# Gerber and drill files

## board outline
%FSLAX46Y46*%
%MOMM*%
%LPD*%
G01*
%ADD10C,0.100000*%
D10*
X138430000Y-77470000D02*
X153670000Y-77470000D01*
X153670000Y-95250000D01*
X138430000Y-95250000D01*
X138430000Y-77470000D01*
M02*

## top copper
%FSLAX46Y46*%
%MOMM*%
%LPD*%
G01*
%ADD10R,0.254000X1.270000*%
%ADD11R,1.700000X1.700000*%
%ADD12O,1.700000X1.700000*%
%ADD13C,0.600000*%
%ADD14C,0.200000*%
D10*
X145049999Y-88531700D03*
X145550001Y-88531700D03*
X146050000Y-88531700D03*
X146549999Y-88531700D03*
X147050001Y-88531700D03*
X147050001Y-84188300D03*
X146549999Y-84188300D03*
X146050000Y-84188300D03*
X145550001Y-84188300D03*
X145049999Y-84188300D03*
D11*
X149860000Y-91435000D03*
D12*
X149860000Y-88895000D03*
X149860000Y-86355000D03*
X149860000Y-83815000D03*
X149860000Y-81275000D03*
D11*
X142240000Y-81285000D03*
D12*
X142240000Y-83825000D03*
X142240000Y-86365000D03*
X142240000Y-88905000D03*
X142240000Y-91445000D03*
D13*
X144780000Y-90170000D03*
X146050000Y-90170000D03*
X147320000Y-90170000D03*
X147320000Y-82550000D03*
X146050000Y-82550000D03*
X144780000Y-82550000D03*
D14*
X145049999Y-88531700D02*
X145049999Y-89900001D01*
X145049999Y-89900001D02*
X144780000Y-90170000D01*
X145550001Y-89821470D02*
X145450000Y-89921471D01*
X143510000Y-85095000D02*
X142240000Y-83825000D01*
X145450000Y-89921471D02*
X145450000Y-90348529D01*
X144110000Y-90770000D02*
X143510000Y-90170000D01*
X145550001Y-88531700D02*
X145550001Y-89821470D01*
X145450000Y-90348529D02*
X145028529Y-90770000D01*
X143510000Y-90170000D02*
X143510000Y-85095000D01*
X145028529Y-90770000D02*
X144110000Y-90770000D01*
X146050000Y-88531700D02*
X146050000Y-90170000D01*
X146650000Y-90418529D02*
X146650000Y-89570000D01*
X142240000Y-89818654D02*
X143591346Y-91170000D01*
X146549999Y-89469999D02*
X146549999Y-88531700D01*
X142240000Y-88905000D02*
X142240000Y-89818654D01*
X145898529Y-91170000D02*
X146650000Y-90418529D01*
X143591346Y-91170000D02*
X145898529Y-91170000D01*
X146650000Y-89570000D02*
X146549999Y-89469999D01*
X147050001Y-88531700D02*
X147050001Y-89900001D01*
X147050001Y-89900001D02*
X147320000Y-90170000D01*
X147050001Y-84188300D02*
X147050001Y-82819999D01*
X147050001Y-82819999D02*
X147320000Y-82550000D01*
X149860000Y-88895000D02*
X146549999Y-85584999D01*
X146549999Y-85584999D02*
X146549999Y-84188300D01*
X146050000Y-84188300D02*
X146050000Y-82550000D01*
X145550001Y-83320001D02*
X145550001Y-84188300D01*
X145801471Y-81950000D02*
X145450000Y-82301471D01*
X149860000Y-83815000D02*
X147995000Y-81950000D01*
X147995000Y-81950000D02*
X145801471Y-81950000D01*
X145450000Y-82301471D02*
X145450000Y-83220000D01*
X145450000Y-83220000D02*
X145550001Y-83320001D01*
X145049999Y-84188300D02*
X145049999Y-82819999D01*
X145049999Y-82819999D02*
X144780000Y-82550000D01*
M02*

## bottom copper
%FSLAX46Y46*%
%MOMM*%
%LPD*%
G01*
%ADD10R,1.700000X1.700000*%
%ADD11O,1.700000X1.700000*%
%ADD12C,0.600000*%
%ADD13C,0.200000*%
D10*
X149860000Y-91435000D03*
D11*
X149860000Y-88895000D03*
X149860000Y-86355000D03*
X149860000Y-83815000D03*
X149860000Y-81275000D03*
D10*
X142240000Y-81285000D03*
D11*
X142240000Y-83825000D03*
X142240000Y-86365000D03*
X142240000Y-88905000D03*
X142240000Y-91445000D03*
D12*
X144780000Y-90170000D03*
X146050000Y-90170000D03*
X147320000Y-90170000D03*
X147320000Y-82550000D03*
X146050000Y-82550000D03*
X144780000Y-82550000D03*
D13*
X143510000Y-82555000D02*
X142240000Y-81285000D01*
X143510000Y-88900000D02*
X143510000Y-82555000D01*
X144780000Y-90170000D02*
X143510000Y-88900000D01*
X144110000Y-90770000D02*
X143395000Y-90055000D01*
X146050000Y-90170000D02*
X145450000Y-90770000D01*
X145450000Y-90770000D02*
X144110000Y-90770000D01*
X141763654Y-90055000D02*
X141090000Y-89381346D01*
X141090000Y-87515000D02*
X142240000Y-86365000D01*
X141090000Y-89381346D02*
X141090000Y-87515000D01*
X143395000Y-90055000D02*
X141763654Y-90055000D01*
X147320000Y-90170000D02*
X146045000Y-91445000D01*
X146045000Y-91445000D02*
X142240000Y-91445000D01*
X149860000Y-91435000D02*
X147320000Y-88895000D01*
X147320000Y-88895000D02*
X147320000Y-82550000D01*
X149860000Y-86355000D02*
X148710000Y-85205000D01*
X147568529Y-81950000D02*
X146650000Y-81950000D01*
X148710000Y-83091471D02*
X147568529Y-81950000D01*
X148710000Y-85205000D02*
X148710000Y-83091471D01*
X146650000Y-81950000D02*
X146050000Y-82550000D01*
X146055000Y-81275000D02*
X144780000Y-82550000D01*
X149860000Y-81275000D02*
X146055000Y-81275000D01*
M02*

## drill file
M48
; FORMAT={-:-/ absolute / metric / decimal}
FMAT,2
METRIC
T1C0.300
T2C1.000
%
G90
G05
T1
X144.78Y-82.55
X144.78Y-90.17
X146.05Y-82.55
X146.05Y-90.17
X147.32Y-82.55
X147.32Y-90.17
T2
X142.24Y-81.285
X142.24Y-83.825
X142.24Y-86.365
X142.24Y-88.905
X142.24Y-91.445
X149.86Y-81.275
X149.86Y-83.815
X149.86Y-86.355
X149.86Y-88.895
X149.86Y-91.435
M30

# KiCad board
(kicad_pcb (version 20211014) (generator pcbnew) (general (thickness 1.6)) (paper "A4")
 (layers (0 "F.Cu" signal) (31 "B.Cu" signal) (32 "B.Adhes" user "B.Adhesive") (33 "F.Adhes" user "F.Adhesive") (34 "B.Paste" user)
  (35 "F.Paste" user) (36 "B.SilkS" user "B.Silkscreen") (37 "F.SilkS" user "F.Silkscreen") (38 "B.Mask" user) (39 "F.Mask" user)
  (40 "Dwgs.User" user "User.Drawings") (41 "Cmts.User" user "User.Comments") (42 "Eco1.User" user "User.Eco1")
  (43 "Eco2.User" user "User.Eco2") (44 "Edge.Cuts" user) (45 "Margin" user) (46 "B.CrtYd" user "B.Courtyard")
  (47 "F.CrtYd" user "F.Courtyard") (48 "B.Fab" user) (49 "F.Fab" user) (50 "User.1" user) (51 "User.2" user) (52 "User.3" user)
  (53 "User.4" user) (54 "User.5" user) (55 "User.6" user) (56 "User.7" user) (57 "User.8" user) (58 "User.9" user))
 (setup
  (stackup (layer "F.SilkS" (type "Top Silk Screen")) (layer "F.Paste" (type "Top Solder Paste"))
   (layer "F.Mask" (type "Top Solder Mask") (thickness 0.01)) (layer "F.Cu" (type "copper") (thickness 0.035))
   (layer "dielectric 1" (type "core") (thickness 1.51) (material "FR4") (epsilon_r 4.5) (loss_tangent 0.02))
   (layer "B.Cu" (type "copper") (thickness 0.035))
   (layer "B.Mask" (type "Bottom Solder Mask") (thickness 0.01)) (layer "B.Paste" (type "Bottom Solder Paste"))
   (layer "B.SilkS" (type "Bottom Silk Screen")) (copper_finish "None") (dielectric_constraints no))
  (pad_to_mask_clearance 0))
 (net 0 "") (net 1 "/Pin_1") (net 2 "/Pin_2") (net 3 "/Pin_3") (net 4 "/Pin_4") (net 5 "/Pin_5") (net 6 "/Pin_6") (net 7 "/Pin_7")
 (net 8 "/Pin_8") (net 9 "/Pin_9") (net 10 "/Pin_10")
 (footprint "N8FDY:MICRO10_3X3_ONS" (layer "F.Cu") (at 146.05 86.36 90)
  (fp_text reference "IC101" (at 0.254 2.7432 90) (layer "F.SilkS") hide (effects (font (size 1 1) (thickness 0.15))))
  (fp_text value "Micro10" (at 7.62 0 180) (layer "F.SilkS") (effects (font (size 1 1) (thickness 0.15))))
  (pad "1" smd rect (at -2.1717 -1.000001 90) (size 1.27 0.254) (layers "F.Cu" "F.Paste" "F.Mask") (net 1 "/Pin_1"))
  (pad "2" smd rect (at -2.1717 -0.499999 90) (size 1.27 0.254) (layers "F.Cu" "F.Paste" "F.Mask") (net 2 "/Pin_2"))
  (pad "3" smd rect (at -2.1717 0 90) (size 1.27 0.254) (layers "F.Cu" "F.Paste" "F.Mask") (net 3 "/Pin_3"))
  (pad "4" smd rect (at -2.1717 0.499999 90) (size 1.27 0.254) (layers "F.Cu" "F.Paste" "F.Mask") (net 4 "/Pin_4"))
  (pad "5" smd rect (at -2.1717 1.000001 90) (size 1.27 0.254) (layers "F.Cu" "F.Paste" "F.Mask") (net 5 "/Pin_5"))
  (pad "6" smd rect (at 2.1717 1.000001 90) (size 1.27 0.254) (layers "F.Cu" "F.Paste" "F.Mask") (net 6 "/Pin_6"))
  (pad "7" smd rect (at 2.1717 0.499999 90) (size 1.27 0.254) (layers "F.Cu" "F.Paste" "F.Mask") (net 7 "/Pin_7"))
  (pad "8" smd rect (at 2.1717 0 90) (size 1.27 0.254) (layers "F.Cu" "F.Paste" "F.Mask") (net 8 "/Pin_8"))
  (pad "9" smd rect (at 2.1717 -0.499999 90) (size 1.27 0.254) (layers "F.Cu" "F.Paste" "F.Mask") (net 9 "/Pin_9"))
  (pad "10" smd rect (at 2.1717 -1.000001 90) (size 1.27 0.254) (layers "F.Cu" "F.Paste" "F.Mask") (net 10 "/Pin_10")))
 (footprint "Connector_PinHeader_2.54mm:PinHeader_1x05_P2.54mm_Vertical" (layer "B.Cu") (at 149.86 91.435)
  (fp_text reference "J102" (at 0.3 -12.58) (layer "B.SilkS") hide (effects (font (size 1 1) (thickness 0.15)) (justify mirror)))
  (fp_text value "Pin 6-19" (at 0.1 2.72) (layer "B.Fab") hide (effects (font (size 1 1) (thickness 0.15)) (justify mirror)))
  (pad "1" thru_hole rect (at 0 0) (size 1.7 1.7) (drill 1) (layers *.Cu *.Mask) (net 6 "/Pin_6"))
  (pad "2" thru_hole oval (at 0 -2.54) (size 1.7 1.7) (drill 1) (layers *.Cu *.Mask) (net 7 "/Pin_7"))
  (pad "3" thru_hole oval (at 0 -5.08) (size 1.7 1.7) (drill 1) (layers *.Cu *.Mask) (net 8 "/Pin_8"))
  (pad "4" thru_hole oval (at 0 -7.62) (size 1.7 1.7) (drill 1) (layers *.Cu *.Mask) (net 9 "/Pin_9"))
  (pad "5" thru_hole oval (at 0 -10.16) (size 1.7 1.7) (drill 1) (layers *.Cu *.Mask) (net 10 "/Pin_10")))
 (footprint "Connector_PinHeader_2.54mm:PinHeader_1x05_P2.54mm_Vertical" (layer "B.Cu") (at 142.24 81.285 180)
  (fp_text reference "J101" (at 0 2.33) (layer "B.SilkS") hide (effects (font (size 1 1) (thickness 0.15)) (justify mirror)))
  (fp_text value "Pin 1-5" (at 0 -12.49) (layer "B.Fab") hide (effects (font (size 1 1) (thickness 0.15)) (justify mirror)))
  (pad "1" thru_hole rect (at 0 0 180) (size 1.7 1.7) (drill 1) (layers *.Cu *.Mask) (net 1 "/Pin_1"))
  (pad "2" thru_hole oval (at 0 -2.54 180) (size 1.7 1.7) (drill 1) (layers *.Cu *.Mask) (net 2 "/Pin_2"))
  (pad "3" thru_hole oval (at 0 -5.08 180) (size 1.7 1.7) (drill 1) (layers *.Cu *.Mask) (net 3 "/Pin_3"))
  (pad "4" thru_hole oval (at 0 -7.62 180) (size 1.7 1.7) (drill 1) (layers *.Cu *.Mask) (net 4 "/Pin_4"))
  (pad "5" thru_hole oval (at 0 -10.16 180) (size 1.7 1.7) (drill 1) (layers *.Cu *.Mask) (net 5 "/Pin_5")))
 (gr_rect (start 138.43 95.25) (end 153.67 77.47) (layer "Edge.Cuts") (width 0.1) (fill none))
 (segment (start 145.049999 88.5317) (end 145.049999 89.900001) (width 0.2) (layer "F.Cu") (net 1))
 (segment (start 145.049999 89.900001) (end 144.78 90.17) (width 0.2) (layer "F.Cu") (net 1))
 (via (at 144.78 90.17) (size 0.6) (drill 0.3) (layers "F.Cu" "B.Cu") (free) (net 1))
 (segment (start 143.51 82.555) (end 142.24 81.285) (width 0.2) (layer "B.Cu") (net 1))
 (segment (start 143.51 88.9) (end 143.51 82.555) (width 0.2) (layer "B.Cu") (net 1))
 (segment (start 144.78 90.17) (end 143.51 88.9) (width 0.2) (layer "B.Cu") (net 1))
 (segment (start 145.550001 89.82147) (end 145.45 89.921471) (width 0.2) (layer "F.Cu") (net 2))
 (segment (start 143.51 85.095) (end 142.24 83.825) (width 0.2) (layer "F.Cu") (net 2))
 (segment (start 145.45 89.921471) (end 145.45 90.348529) (width 0.2) (layer "F.Cu") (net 2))
 (segment (start 144.11 90.77) (end 143.51 90.17) (width 0.2) (layer "F.Cu") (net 2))
 (segment (start 145.550001 88.5317) (end 145.550001 89.82147) (width 0.2) (layer "F.Cu") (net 2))
 (segment (start 145.45 90.348529) (end 145.028529 90.77) (width 0.2) (layer "F.Cu") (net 2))
 (segment (start 143.51 90.17) (end 143.51 85.095) (width 0.2) (layer "F.Cu") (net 2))
 (segment (start 145.028529 90.77) (end 144.11 90.77) (width 0.2) (layer "F.Cu") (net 2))
 (segment (start 146.05 88.5317) (end 146.05 90.17) (width 0.2) (layer "F.Cu") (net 3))
 (via (at 146.05 90.17) (size 0.6) (drill 0.3) (layers "F.Cu" "B.Cu") (free) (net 3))
 (segment (start 144.11 90.77) (end 143.395 90.055) (width 0.2) (layer "B.Cu") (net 3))
 (segment (start 146.05 90.17) (end 145.45 90.77) (width 0.2) (layer "B.Cu") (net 3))
 (segment (start 145.45 90.77) (end 144.11 90.77) (width 0.2) (layer "B.Cu") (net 3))
 (segment (start 141.763654 90.055) (end 141.09 89.381346) (width 0.2) (layer "B.Cu") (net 3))
 (segment (start 141.09 87.515) (end 142.24 86.365) (width 0.2) (layer "B.Cu") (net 3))
 (segment (start 141.09 89.381346) (end 141.09 87.515) (width 0.2) (layer "B.Cu") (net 3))
 (segment (start 143.395 90.055) (end 141.763654 90.055) (width 0.2) (layer "B.Cu") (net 3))
 (segment (start 146.65 90.418529) (end 146.65 89.57) (width 0.2) (layer "F.Cu") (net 4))
 (segment (start 142.24 89.818654) (end 143.591346 91.17) (width 0.2) (layer "F.Cu") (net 4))
 (segment (start 146.549999 89.469999) (end 146.549999 88.5317) (width 0.2) (layer "F.Cu") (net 4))
 (segment (start 142.24 88.905) (end 142.24 89.818654) (width 0.2) (layer "F.Cu") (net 4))
 (segment (start 145.898529 91.17) (end 146.65 90.418529) (width 0.2) (layer "F.Cu") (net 4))
 (segment (start 143.591346 91.17) (end 145.898529 91.17) (width 0.2) (layer "F.Cu") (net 4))
 (segment (start 146.65 89.57) (end 146.549999 89.469999) (width 0.2) (layer "F.Cu") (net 4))
 (segment (start 147.050001 88.5317) (end 147.050001 89.900001) (width 0.2) (layer "F.Cu") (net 5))
 (segment (start 147.050001 89.900001) (end 147.32 90.17) (width 0.2) (layer "F.Cu") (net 5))
 (via (at 147.32 90.17) (size 0.6) (drill 0.3) (layers "F.Cu" "B.Cu") (free) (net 5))
 (segment (start 147.32 90.17) (end 146.045 91.445) (width 0.2) (layer "B.Cu") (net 5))
 (segment (start 146.045 91.445) (end 142.24 91.445) (width 0.2) (layer "B.Cu") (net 5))
 (segment (start 147.050001 84.1883) (end 147.050001 82.819999) (width 0.2) (layer "F.Cu") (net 6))
 (segment (start 147.050001 82.819999) (end 147.32 82.55) (width 0.2) (layer "F.Cu") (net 6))
 (via (at 147.32 82.55) (size 0.6) (drill 0.3) (layers "F.Cu" "B.Cu") (free) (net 6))
 (segment (start 149.86 91.435) (end 147.32 88.895) (width 0.2) (layer "B.Cu") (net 6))
 (segment (start 147.32 88.895) (end 147.32 82.55) (width 0.2) (layer "B.Cu") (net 6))
 (segment (start 149.86 88.895) (end 146.549999 85.584999) (width 0.2) (layer "F.Cu") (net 7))
 (segment (start 146.549999 85.584999) (end 146.549999 84.1883) (width 0.2) (layer "F.Cu") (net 7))
 (segment (start 146.05 84.1883) (end 146.05 82.55) (width 0.2) (layer "F.Cu") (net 8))
 (via (at 146.05 82.55) (size 0.6) (drill 0.3) (layers "F.Cu" "B.Cu") (free) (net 8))
 (segment (start 149.86 86.355) (end 148.71 85.205) (width 0.2) (layer "B.Cu") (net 8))
 (segment (start 147.568529 81.95) (end 146.65 81.95) (width 0.2) (layer "B.Cu") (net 8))
 (segment (start 148.71 83.091471) (end 147.568529 81.95) (width 0.2) (layer "B.Cu") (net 8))
 (segment (start 148.71 85.205) (end 148.71 83.091471) (width 0.2) (layer "B.Cu") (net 8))
 (segment (start 146.65 81.95) (end 146.05 82.55) (width 0.2) (layer "B.Cu") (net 8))
 (segment (start 145.550001 83.320001) (end 145.550001 84.1883) (width 0.2) (layer "F.Cu") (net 9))
 (segment (start 145.801471 81.95) (end 145.45 82.301471) (width 0.2) (layer "F.Cu") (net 9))
 (segment (start 149.86 83.815) (end 147.995 81.95) (width 0.2) (layer "F.Cu") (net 9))
 (segment (start 147.995 81.95) (end 145.801471 81.95) (width 0.2) (layer "F.Cu") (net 9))
 (segment (start 145.45 82.301471) (end 145.45 83.22) (width 0.2) (layer "F.Cu") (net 9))
 (segment (start 145.45 83.22) (end 145.550001 83.320001) (width 0.2) (layer "F.Cu") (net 9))
 (segment (start 145.049999 84.1883) (end 145.049999 82.819999) (width 0.2) (layer "F.Cu") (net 10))
 (segment (start 145.049999 82.819999) (end 144.78 82.55) (width 0.2) (layer "F.Cu") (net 10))
 (via (at 144.78 82.55) (size 0.6) (drill 0.3) (layers "F.Cu" "B.Cu") (free) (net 10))
 (segment (start 146.055 81.275) (end 144.78 82.55) (width 0.2) (layer "B.Cu") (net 10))
 (segment (start 149.86 81.275) (end 146.055 81.275) (width 0.2) (layer "B.Cu") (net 10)))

